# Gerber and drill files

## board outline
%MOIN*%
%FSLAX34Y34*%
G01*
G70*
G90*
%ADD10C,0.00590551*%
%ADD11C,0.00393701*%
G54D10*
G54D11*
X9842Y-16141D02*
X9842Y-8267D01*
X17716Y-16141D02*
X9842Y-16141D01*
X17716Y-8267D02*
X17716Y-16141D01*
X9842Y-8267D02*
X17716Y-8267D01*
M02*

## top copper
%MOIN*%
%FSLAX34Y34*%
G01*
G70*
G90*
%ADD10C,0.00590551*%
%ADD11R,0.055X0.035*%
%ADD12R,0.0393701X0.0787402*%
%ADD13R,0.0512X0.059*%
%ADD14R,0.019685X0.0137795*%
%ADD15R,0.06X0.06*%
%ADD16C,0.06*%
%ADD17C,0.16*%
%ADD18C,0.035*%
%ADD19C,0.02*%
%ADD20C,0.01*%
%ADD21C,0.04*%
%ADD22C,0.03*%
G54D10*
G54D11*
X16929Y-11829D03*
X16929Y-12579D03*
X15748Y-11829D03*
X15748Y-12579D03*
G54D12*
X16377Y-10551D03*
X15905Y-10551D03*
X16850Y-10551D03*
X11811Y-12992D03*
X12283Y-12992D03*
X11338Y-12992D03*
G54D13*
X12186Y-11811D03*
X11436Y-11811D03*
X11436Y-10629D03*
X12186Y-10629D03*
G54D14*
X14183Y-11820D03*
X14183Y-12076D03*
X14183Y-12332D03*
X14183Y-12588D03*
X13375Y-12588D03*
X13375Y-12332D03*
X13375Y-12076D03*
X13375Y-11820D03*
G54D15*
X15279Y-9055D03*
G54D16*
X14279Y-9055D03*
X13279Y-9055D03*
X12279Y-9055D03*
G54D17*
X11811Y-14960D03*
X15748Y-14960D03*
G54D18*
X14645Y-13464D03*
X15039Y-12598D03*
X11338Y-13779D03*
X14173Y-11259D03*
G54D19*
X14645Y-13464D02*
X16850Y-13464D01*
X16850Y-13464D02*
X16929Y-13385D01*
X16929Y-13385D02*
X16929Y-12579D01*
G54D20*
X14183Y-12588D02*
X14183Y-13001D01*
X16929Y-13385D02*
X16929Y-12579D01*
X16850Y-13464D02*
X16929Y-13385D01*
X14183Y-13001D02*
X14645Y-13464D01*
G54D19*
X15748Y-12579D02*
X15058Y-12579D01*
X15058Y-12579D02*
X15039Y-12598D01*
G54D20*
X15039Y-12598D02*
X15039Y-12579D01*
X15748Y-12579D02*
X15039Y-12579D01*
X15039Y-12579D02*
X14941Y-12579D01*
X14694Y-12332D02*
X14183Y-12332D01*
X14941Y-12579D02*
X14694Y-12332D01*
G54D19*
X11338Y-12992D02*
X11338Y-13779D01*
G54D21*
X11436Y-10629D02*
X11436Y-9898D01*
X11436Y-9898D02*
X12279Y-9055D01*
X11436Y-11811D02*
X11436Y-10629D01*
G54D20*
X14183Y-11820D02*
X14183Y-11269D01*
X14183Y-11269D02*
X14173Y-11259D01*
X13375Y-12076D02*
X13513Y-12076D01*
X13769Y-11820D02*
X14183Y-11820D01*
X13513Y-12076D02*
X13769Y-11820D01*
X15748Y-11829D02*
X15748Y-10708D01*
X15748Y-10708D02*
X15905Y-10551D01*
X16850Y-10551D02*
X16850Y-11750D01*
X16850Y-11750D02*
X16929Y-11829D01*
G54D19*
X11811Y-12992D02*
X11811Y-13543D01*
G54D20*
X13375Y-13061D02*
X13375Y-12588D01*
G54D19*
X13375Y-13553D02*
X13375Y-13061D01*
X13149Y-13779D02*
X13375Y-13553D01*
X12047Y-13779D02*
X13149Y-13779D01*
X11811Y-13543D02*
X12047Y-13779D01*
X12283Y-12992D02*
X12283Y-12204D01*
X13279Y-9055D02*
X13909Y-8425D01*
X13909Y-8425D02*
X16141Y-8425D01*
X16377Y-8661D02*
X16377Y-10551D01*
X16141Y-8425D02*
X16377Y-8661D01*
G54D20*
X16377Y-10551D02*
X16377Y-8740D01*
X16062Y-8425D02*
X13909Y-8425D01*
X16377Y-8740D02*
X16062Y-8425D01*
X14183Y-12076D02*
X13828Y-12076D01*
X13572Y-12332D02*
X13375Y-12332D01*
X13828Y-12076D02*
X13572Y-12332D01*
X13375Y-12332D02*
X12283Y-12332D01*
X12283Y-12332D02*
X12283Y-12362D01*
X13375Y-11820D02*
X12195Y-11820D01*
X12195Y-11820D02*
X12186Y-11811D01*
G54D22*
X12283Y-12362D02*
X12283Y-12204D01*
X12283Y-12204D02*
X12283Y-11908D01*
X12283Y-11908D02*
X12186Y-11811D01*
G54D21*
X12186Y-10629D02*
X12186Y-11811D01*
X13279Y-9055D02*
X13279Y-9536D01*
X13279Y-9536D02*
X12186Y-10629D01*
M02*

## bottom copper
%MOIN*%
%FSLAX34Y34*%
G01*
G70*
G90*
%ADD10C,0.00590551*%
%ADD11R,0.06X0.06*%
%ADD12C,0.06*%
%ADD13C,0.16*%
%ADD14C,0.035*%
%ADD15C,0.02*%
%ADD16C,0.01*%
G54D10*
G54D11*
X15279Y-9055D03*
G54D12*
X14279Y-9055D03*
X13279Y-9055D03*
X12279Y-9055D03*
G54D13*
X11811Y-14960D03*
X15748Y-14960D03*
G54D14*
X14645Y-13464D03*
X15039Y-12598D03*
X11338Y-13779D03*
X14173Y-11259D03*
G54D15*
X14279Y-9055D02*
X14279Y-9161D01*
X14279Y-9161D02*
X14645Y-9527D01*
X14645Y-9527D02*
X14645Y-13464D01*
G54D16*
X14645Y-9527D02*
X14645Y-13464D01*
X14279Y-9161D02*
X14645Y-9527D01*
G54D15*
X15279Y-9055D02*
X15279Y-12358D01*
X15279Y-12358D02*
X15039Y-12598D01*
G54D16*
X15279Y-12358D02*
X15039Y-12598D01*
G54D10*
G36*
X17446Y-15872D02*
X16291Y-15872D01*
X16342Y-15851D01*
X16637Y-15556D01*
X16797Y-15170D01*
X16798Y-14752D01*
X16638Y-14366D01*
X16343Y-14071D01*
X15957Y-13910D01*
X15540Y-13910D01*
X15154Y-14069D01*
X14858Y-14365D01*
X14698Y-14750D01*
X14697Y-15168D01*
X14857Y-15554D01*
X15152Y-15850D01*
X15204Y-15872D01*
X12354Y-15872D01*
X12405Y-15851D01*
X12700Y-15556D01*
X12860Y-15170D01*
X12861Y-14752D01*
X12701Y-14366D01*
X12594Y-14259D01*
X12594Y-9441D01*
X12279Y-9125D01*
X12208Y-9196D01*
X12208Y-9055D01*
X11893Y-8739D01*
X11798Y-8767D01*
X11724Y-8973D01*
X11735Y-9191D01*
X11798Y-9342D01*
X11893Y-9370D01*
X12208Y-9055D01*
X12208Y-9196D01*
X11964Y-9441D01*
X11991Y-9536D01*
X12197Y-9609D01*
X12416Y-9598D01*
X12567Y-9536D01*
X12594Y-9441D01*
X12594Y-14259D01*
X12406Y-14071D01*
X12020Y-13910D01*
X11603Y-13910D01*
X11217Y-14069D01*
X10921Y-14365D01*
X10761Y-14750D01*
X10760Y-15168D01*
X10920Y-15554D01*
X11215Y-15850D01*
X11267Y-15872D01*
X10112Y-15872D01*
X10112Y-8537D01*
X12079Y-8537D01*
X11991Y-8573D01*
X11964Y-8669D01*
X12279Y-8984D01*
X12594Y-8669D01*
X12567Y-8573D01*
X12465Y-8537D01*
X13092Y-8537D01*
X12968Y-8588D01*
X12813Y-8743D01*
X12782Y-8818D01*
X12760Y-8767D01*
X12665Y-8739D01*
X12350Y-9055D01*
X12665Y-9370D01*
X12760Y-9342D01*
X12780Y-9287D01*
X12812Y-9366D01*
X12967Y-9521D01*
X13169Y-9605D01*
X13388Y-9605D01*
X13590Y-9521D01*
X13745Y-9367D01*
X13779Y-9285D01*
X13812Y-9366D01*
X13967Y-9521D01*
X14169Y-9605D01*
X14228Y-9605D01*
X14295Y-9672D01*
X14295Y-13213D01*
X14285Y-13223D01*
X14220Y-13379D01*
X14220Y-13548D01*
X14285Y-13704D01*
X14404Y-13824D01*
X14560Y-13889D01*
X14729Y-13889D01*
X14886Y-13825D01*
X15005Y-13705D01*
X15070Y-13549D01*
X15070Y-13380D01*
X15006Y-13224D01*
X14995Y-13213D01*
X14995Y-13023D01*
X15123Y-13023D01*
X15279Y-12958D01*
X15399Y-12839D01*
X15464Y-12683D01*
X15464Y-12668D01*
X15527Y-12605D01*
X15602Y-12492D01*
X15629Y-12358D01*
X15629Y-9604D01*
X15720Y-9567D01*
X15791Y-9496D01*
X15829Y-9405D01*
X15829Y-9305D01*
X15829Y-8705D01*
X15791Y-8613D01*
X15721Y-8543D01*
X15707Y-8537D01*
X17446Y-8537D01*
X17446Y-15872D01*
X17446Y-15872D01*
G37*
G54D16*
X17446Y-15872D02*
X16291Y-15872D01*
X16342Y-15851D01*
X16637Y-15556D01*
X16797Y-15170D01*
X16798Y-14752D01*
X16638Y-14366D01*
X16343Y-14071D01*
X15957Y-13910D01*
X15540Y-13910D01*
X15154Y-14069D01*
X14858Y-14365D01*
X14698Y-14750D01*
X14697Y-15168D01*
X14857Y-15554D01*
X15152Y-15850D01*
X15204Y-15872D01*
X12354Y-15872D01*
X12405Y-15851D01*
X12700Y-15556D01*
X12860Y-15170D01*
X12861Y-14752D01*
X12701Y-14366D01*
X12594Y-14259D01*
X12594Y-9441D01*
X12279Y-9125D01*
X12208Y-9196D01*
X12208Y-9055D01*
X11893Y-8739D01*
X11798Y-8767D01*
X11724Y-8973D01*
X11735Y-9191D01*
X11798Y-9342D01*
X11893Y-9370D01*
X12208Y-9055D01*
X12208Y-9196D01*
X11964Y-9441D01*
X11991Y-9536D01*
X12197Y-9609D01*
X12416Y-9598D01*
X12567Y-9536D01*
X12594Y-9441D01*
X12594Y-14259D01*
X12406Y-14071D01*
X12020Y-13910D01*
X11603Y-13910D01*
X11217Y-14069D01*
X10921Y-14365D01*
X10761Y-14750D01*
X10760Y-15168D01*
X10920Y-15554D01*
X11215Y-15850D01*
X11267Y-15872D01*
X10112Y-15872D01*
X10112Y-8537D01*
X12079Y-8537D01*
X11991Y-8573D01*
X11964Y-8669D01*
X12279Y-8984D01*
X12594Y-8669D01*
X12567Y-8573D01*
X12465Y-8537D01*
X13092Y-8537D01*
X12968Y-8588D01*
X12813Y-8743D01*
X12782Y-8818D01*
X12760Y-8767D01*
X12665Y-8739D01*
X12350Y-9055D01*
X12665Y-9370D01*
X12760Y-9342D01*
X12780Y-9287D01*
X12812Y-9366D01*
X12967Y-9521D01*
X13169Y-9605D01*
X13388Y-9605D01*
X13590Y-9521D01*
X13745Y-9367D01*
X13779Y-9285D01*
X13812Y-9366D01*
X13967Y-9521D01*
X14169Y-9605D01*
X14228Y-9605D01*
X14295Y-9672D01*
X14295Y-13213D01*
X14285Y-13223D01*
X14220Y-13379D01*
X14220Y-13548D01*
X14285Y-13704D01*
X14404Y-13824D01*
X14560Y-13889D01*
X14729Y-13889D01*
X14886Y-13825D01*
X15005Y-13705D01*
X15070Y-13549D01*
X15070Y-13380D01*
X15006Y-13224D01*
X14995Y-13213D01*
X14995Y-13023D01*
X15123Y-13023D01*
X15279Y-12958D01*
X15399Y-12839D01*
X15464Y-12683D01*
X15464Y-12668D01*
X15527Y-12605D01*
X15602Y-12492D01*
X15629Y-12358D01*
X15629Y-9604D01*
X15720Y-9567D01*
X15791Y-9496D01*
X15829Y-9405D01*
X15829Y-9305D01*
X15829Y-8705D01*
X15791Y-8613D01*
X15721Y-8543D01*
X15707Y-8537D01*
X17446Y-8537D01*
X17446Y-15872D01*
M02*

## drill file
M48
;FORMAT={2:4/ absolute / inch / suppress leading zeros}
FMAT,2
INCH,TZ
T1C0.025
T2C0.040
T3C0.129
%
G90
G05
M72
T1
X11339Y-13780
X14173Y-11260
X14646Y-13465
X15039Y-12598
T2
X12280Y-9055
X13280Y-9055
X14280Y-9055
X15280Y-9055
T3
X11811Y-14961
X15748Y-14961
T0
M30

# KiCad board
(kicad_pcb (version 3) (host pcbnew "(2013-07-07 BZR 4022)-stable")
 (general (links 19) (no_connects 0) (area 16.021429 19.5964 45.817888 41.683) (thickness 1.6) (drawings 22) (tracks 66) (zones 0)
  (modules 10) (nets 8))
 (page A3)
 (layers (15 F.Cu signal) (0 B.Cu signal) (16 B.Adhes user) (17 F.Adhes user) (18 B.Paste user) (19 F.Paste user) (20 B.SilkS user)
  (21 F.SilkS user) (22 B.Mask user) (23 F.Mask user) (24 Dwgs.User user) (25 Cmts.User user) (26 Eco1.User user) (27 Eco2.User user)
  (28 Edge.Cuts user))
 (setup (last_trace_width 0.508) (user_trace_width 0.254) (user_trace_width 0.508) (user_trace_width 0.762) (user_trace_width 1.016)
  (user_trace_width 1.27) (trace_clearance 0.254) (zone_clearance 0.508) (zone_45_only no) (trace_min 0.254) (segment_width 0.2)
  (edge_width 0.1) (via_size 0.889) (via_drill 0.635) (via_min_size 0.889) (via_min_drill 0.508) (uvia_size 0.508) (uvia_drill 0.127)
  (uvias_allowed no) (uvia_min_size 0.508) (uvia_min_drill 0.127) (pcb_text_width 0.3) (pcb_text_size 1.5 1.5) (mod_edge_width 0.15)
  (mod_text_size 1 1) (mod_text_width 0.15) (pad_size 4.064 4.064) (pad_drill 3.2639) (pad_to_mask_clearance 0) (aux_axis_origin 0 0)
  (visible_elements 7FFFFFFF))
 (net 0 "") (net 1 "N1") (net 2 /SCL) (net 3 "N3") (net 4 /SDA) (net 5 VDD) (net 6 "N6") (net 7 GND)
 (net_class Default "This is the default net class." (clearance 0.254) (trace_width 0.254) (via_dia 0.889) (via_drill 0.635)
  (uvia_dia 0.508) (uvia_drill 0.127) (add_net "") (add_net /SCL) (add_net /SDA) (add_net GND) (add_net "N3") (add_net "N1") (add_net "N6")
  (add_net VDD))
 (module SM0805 (layer F.Cu) (at 43 31 270)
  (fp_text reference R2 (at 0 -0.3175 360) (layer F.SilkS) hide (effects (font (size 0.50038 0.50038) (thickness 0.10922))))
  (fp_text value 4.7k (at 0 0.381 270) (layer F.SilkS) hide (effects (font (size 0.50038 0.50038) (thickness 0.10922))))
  (pad 1 smd rect (at -0.9525 0 270) (size 0.889 1.397) (layers F.Cu F.Paste F.Mask) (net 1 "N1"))
  (pad 2 smd rect (at 0.9525 0 270) (size 0.889 1.397) (layers F.Cu F.Paste F.Mask) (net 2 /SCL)))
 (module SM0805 (layer F.Cu) (at 40 31 270)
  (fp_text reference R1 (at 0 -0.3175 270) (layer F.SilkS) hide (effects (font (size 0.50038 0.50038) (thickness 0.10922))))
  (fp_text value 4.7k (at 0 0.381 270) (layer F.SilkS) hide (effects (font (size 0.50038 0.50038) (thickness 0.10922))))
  (pad 1 smd rect (at -0.9525 0 270) (size 0.889 1.397) (layers F.Cu F.Paste F.Mask) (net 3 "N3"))
  (pad 2 smd rect (at 0.9525 0 270) (size 0.889 1.397) (layers F.Cu F.Paste F.Mask) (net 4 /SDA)))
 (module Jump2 (layer F.Cu) (at 41.6 26.8)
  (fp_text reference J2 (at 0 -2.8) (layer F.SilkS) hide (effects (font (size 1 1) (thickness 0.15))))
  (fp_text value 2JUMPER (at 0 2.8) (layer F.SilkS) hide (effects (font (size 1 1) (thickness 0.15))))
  (pad 1 smd rect (at 0 0) (size 1 2) (layers F.Cu F.Paste F.Mask) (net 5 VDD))
  (pad 2 smd rect (at -1.2 0) (size 1 2) (layers F.Cu F.Paste F.Mask) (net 3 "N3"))
  (pad 3 smd rect (at 1.2 0 180) (size 1 2) (layers F.Cu F.Paste F.Mask) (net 1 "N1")))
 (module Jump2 (layer F.Cu) (at 30 33 180)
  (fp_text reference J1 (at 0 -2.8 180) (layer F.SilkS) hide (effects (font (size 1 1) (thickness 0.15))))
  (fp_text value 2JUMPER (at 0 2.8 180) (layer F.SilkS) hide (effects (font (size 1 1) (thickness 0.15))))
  (pad 1 smd rect (at 0 0 180) (size 1 2) (layers F.Cu F.Paste F.Mask) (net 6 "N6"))
  (pad 2 smd rect (at -1.2 0 180) (size 1 2) (layers F.Cu F.Paste F.Mask) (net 5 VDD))
  (pad 3 smd rect (at 1.2 0) (size 1 2) (layers F.Cu F.Paste F.Mask) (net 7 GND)))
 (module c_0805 (layer F.Cu) (at 30 30)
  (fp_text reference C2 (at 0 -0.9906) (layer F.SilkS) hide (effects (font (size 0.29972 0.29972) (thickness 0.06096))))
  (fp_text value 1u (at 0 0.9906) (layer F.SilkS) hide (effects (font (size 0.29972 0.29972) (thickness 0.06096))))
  (pad 1 smd rect (at 0.9525 0) (size 1.30048 1.4986) (layers F.Cu F.Paste F.Mask) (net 5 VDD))
  (pad 2 smd rect (at -0.9525 0) (size 1.30048 1.4986) (layers F.Cu F.Paste F.Mask) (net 7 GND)))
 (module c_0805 (layer F.Cu) (at 30 27 180)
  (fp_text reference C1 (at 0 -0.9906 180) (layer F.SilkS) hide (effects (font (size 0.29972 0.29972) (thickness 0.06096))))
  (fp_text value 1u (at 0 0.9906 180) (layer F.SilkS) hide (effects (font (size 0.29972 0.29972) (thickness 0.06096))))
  (pad 1 smd rect (at 0.9525 0 180) (size 1.30048 1.4986) (layers F.Cu F.Paste F.Mask) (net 7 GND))
  (pad 2 smd rect (at -0.9525 0 180) (size 1.30048 1.4986) (layers F.Cu F.Paste F.Mask) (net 5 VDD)))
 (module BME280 (layer F.Cu) (at 35 31)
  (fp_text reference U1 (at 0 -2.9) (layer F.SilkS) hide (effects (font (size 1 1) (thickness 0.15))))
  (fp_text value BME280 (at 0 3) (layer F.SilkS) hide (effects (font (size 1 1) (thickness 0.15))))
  (pad 1 smd rect (at 1.025 -0.975) (size 0.5 0.35) (layers F.Cu F.Paste F.Mask) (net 7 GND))
  (pad 2 smd rect (at 1.025 -0.325) (size 0.5 0.35) (layers F.Cu F.Paste F.Mask) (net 5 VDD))
  (pad 3 smd rect (at 1.025 0.325) (size 0.5 0.35) (layers F.Cu F.Paste F.Mask) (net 4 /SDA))
  (pad 4 smd rect (at 1.025 0.975) (size 0.5 0.35) (layers F.Cu F.Paste F.Mask) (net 2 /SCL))
  (pad 5 smd rect (at -1.025 0.975) (size 0.5 0.35) (layers F.Cu F.Paste F.Mask) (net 6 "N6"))
  (pad 6 smd rect (at -1.025 0.325) (size 0.5 0.35) (layers F.Cu F.Paste F.Mask) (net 5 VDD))
  (pad 7 smd rect (at -1.025 -0.325) (size 0.5 0.35) (layers F.Cu F.Paste F.Mask) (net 7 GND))
  (pad 8 smd rect (at -1.025 -0.975) (size 0.5 0.35) (layers F.Cu F.Paste F.Mask) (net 5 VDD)))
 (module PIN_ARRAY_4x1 (layer F.Cu) (at 35 23 180)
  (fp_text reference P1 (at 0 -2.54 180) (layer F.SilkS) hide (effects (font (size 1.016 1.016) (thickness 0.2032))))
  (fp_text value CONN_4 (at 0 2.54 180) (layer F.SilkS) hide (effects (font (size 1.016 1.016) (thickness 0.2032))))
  (pad 1 thru_hole rect (at -3.81 0 180) (size 1.524 1.524) (drill 1.016) (layers *.Cu *.Mask F.SilkS) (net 4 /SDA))
  (pad 2 thru_hole circle (at -1.27 0 180) (size 1.524 1.524) (drill 1.016) (layers *.Cu *.Mask F.SilkS) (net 2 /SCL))
  (pad 3 thru_hole circle (at 1.27 0 180) (size 1.524 1.524) (drill 1.016) (layers *.Cu *.Mask F.SilkS) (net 5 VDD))
  (pad 4 thru_hole circle (at 3.81 0 180) (size 1.524 1.524) (drill 1.016) (layers *.Cu *.Mask F.SilkS) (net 7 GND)))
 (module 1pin (layer F.Cu) (at 30 38 90)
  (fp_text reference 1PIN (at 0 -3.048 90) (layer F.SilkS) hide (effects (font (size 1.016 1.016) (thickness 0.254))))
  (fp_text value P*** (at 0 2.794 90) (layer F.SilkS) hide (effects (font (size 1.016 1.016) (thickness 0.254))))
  (pad 1 thru_hole circle (at 0 0 90) (size 4.064 4.064) (drill 3.2639) (layers *.Cu *.Mask F.SilkS)))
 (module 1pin (layer F.Cu) (at 40 38)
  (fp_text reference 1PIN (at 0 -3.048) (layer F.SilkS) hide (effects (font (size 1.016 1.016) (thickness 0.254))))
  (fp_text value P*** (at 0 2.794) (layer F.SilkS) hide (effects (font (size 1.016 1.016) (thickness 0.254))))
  (pad 1 thru_hole circle (at 0 0) (size 4.064 4.064) (drill 3.2639) (layers *.Cu *.Mask F.SilkS)))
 (gr_line (start 25 41) (end 25 21) (angle 90) (layer Edge.Cuts) (width 0.1))
 (gr_line (start 45 41) (end 25 41) (angle 90) (layer Edge.Cuts) (width 0.1))
 (gr_line (start 45 21) (end 45 41) (angle 90) (layer Edge.Cuts) (width 0.1))
 (gr_line (start 25 21) (end 45 21) (angle 90) (layer Edge.Cuts) (width 0.1))
 (segment (start 36.27 23) (end 36.27 23.27) (width 0.508) (layer B.Cu) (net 2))
 (segment (start 36.27 23.27) (end 37.2 24.2) (width 0.508) (layer B.Cu) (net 2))
 (segment (start 37.2 24.2) (end 37.2 34.2) (width 0.508) (layer B.Cu) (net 2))
 (segment (start 37.2 34.2) (end 42.8 34.2) (width 0.508) (layer F.Cu) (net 2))
 (segment (start 42.8 34.2) (end 43 34) (width 0.508) (layer F.Cu) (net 2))
 (segment (start 43 34) (end 43 31.9525) (width 0.508) (layer F.Cu) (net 2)) (via (at 37.2 34.2) (size 0.889) (layers F.Cu B.Cu) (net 2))
 (segment (start 37.2 24.2) (end 37.2 34.2) (width 0.254) (layer B.Cu) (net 2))
 (segment (start 36.27 23.27) (end 37.2 24.2) (width 0.254) (layer B.Cu) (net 2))
 (segment (start 36.025 31.975) (end 36.025 33.025) (width 0.254) (layer F.Cu) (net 2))
 (segment (start 43 34) (end 43 31.9525) (width 0.254) (layer F.Cu) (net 2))
 (segment (start 42.8 34.2) (end 43 34) (width 0.254) (layer F.Cu) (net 2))
 (segment (start 36.025 33.025) (end 37.2 34.2) (width 0.254) (layer F.Cu) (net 2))
 (segment (start 38.81 23) (end 38.81 31.39) (width 0.508) (layer B.Cu) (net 4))
 (segment (start 38.81 31.39) (end 38.2 32) (width 0.508) (layer B.Cu) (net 4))
 (segment (start 40 31.9525) (end 38.2475 31.9525) (width 0.508) (layer F.Cu) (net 4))
 (segment (start 38.2475 31.9525) (end 38.2 32) (width 0.508) (layer F.Cu) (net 4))
 (segment (start 38.81 31.39) (end 38.2 32) (width 0.254) (layer B.Cu) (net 4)) (via (at 38.2 32) (size 0.889) (layers F.Cu B.Cu) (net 4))
 (segment (start 38.2 32) (end 38.2 31.9525) (width 0.254) (layer F.Cu) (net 4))
 (segment (start 40 31.9525) (end 38.2 31.9525) (width 0.254) (layer F.Cu) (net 4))
 (segment (start 38.2 31.9525) (end 37.9525 31.9525) (width 0.254) (layer F.Cu) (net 4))
 (segment (start 37.325 31.325) (end 36.025 31.325) (width 0.254) (layer F.Cu) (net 4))
 (segment (start 37.9525 31.9525) (end 37.325 31.325) (width 0.254) (layer F.Cu) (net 4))
 (segment (start 28.8 33) (end 28.8 35) (width 0.508) (layer F.Cu) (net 7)) (via (at 28.8 35) (size 0.889) (layers F.Cu B.Cu) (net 7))
 (segment (start 29.0475 27) (end 29.0475 25.1425) (width 1.016) (layer F.Cu) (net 7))
 (segment (start 29.0475 25.1425) (end 31.19 23) (width 1.016) (layer F.Cu) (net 7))
 (segment (start 29.0475 30) (end 29.0475 27) (width 1.016) (layer F.Cu) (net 7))
 (segment (start 36.025 30.025) (end 36.025 28.625) (width 0.254) (layer F.Cu) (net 7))
 (via (at 36 28.6) (size 0.889) (layers F.Cu B.Cu) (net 7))
 (segment (start 36.025 28.625) (end 36 28.6) (width 0.254) (layer F.Cu) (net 7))
 (segment (start 33.975 30.675) (end 34.325 30.675) (width 0.254) (layer F.Cu) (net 7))
 (segment (start 34.975 30.025) (end 36.025 30.025) (width 0.254) (layer F.Cu) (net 7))
 (segment (start 34.325 30.675) (end 34.975 30.025) (width 0.254) (layer F.Cu) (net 7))
 (segment (start 40 30.0475) (end 40 27.2) (width 0.254) (layer F.Cu) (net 3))
 (segment (start 40 27.2) (end 40.4 26.8) (width 0.254) (layer F.Cu) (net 3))
 (segment (start 42.8 26.8) (end 42.8 29.8475) (width 0.254) (layer F.Cu) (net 1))
 (segment (start 42.8 29.8475) (end 43 30.0475) (width 0.254) (layer F.Cu) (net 1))
 (segment (start 30 33) (end 30 34.4) (width 0.508) (layer F.Cu) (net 6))
 (segment (start 33.975 33.175) (end 33.975 31.975) (width 0.254) (layer F.Cu) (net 6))
 (segment (start 33.975 34.425) (end 33.975 33.175) (width 0.508) (layer F.Cu) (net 6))
 (segment (start 33.4 35) (end 33.975 34.425) (width 0.508) (layer F.Cu) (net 6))
 (segment (start 30.6 35) (end 33.4 35) (width 0.508) (layer F.Cu) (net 6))
 (segment (start 30 34.4) (end 30.6 35) (width 0.508) (layer F.Cu) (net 6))
 (segment (start 31.2 33) (end 31.2 31) (width 0.508) (layer F.Cu) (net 5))
 (segment (start 33.73 23) (end 35.33 21.4) (width 0.508) (layer F.Cu) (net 5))
 (segment (start 35.33 21.4) (end 41 21.4) (width 0.508) (layer F.Cu) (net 5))
 (segment (start 41.6 22) (end 41.6 26.8) (width 0.508) (layer F.Cu) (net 5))
 (segment (start 41 21.4) (end 41.6 22) (width 0.508) (layer F.Cu) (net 5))
 (segment (start 41.6 26.8) (end 41.6 22.2) (width 0.254) (layer F.Cu) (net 5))
 (segment (start 40.8 21.4) (end 35.33 21.4) (width 0.254) (layer F.Cu) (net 5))
 (segment (start 41.6 22.2) (end 40.8 21.4) (width 0.254) (layer F.Cu) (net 5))
 (segment (start 36.025 30.675) (end 35.125 30.675) (width 0.254) (layer F.Cu) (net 5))
 (segment (start 34.475 31.325) (end 33.975 31.325) (width 0.254) (layer F.Cu) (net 5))
 (segment (start 35.125 30.675) (end 34.475 31.325) (width 0.254) (layer F.Cu) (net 5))
 (segment (start 33.975 31.325) (end 31.2 31.325) (width 0.254) (layer F.Cu) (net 5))
 (segment (start 31.2 31.325) (end 31.2 31.4) (width 0.254) (layer F.Cu) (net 5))
 (segment (start 33.975 30.025) (end 30.9775 30.025) (width 0.254) (layer F.Cu) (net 5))
 (segment (start 30.9775 30.025) (end 30.9525 30) (width 0.254) (layer F.Cu) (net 5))
 (segment (start 31.2 31.4) (end 31.2 31) (width 0.762) (layer F.Cu) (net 5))
 (segment (start 31.2 31) (end 31.2 30.2475) (width 0.762) (layer F.Cu) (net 5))
 (segment (start 31.2 30.2475) (end 30.9525 30) (width 0.762) (layer F.Cu) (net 5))
 (segment (start 30.9525 27) (end 30.9525 30) (width 1.016) (layer F.Cu) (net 5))
 (segment (start 33.73 23) (end 33.73 24.2225) (width 1.016) (layer F.Cu) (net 5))
 (segment (start 33.73 24.2225) (end 30.9525 27) (width 1.016) (layer F.Cu) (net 5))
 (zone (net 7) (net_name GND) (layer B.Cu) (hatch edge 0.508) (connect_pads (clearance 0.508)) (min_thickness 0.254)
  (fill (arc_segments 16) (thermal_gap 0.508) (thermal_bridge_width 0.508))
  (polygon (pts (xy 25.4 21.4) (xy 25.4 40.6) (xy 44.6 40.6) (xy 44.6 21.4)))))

